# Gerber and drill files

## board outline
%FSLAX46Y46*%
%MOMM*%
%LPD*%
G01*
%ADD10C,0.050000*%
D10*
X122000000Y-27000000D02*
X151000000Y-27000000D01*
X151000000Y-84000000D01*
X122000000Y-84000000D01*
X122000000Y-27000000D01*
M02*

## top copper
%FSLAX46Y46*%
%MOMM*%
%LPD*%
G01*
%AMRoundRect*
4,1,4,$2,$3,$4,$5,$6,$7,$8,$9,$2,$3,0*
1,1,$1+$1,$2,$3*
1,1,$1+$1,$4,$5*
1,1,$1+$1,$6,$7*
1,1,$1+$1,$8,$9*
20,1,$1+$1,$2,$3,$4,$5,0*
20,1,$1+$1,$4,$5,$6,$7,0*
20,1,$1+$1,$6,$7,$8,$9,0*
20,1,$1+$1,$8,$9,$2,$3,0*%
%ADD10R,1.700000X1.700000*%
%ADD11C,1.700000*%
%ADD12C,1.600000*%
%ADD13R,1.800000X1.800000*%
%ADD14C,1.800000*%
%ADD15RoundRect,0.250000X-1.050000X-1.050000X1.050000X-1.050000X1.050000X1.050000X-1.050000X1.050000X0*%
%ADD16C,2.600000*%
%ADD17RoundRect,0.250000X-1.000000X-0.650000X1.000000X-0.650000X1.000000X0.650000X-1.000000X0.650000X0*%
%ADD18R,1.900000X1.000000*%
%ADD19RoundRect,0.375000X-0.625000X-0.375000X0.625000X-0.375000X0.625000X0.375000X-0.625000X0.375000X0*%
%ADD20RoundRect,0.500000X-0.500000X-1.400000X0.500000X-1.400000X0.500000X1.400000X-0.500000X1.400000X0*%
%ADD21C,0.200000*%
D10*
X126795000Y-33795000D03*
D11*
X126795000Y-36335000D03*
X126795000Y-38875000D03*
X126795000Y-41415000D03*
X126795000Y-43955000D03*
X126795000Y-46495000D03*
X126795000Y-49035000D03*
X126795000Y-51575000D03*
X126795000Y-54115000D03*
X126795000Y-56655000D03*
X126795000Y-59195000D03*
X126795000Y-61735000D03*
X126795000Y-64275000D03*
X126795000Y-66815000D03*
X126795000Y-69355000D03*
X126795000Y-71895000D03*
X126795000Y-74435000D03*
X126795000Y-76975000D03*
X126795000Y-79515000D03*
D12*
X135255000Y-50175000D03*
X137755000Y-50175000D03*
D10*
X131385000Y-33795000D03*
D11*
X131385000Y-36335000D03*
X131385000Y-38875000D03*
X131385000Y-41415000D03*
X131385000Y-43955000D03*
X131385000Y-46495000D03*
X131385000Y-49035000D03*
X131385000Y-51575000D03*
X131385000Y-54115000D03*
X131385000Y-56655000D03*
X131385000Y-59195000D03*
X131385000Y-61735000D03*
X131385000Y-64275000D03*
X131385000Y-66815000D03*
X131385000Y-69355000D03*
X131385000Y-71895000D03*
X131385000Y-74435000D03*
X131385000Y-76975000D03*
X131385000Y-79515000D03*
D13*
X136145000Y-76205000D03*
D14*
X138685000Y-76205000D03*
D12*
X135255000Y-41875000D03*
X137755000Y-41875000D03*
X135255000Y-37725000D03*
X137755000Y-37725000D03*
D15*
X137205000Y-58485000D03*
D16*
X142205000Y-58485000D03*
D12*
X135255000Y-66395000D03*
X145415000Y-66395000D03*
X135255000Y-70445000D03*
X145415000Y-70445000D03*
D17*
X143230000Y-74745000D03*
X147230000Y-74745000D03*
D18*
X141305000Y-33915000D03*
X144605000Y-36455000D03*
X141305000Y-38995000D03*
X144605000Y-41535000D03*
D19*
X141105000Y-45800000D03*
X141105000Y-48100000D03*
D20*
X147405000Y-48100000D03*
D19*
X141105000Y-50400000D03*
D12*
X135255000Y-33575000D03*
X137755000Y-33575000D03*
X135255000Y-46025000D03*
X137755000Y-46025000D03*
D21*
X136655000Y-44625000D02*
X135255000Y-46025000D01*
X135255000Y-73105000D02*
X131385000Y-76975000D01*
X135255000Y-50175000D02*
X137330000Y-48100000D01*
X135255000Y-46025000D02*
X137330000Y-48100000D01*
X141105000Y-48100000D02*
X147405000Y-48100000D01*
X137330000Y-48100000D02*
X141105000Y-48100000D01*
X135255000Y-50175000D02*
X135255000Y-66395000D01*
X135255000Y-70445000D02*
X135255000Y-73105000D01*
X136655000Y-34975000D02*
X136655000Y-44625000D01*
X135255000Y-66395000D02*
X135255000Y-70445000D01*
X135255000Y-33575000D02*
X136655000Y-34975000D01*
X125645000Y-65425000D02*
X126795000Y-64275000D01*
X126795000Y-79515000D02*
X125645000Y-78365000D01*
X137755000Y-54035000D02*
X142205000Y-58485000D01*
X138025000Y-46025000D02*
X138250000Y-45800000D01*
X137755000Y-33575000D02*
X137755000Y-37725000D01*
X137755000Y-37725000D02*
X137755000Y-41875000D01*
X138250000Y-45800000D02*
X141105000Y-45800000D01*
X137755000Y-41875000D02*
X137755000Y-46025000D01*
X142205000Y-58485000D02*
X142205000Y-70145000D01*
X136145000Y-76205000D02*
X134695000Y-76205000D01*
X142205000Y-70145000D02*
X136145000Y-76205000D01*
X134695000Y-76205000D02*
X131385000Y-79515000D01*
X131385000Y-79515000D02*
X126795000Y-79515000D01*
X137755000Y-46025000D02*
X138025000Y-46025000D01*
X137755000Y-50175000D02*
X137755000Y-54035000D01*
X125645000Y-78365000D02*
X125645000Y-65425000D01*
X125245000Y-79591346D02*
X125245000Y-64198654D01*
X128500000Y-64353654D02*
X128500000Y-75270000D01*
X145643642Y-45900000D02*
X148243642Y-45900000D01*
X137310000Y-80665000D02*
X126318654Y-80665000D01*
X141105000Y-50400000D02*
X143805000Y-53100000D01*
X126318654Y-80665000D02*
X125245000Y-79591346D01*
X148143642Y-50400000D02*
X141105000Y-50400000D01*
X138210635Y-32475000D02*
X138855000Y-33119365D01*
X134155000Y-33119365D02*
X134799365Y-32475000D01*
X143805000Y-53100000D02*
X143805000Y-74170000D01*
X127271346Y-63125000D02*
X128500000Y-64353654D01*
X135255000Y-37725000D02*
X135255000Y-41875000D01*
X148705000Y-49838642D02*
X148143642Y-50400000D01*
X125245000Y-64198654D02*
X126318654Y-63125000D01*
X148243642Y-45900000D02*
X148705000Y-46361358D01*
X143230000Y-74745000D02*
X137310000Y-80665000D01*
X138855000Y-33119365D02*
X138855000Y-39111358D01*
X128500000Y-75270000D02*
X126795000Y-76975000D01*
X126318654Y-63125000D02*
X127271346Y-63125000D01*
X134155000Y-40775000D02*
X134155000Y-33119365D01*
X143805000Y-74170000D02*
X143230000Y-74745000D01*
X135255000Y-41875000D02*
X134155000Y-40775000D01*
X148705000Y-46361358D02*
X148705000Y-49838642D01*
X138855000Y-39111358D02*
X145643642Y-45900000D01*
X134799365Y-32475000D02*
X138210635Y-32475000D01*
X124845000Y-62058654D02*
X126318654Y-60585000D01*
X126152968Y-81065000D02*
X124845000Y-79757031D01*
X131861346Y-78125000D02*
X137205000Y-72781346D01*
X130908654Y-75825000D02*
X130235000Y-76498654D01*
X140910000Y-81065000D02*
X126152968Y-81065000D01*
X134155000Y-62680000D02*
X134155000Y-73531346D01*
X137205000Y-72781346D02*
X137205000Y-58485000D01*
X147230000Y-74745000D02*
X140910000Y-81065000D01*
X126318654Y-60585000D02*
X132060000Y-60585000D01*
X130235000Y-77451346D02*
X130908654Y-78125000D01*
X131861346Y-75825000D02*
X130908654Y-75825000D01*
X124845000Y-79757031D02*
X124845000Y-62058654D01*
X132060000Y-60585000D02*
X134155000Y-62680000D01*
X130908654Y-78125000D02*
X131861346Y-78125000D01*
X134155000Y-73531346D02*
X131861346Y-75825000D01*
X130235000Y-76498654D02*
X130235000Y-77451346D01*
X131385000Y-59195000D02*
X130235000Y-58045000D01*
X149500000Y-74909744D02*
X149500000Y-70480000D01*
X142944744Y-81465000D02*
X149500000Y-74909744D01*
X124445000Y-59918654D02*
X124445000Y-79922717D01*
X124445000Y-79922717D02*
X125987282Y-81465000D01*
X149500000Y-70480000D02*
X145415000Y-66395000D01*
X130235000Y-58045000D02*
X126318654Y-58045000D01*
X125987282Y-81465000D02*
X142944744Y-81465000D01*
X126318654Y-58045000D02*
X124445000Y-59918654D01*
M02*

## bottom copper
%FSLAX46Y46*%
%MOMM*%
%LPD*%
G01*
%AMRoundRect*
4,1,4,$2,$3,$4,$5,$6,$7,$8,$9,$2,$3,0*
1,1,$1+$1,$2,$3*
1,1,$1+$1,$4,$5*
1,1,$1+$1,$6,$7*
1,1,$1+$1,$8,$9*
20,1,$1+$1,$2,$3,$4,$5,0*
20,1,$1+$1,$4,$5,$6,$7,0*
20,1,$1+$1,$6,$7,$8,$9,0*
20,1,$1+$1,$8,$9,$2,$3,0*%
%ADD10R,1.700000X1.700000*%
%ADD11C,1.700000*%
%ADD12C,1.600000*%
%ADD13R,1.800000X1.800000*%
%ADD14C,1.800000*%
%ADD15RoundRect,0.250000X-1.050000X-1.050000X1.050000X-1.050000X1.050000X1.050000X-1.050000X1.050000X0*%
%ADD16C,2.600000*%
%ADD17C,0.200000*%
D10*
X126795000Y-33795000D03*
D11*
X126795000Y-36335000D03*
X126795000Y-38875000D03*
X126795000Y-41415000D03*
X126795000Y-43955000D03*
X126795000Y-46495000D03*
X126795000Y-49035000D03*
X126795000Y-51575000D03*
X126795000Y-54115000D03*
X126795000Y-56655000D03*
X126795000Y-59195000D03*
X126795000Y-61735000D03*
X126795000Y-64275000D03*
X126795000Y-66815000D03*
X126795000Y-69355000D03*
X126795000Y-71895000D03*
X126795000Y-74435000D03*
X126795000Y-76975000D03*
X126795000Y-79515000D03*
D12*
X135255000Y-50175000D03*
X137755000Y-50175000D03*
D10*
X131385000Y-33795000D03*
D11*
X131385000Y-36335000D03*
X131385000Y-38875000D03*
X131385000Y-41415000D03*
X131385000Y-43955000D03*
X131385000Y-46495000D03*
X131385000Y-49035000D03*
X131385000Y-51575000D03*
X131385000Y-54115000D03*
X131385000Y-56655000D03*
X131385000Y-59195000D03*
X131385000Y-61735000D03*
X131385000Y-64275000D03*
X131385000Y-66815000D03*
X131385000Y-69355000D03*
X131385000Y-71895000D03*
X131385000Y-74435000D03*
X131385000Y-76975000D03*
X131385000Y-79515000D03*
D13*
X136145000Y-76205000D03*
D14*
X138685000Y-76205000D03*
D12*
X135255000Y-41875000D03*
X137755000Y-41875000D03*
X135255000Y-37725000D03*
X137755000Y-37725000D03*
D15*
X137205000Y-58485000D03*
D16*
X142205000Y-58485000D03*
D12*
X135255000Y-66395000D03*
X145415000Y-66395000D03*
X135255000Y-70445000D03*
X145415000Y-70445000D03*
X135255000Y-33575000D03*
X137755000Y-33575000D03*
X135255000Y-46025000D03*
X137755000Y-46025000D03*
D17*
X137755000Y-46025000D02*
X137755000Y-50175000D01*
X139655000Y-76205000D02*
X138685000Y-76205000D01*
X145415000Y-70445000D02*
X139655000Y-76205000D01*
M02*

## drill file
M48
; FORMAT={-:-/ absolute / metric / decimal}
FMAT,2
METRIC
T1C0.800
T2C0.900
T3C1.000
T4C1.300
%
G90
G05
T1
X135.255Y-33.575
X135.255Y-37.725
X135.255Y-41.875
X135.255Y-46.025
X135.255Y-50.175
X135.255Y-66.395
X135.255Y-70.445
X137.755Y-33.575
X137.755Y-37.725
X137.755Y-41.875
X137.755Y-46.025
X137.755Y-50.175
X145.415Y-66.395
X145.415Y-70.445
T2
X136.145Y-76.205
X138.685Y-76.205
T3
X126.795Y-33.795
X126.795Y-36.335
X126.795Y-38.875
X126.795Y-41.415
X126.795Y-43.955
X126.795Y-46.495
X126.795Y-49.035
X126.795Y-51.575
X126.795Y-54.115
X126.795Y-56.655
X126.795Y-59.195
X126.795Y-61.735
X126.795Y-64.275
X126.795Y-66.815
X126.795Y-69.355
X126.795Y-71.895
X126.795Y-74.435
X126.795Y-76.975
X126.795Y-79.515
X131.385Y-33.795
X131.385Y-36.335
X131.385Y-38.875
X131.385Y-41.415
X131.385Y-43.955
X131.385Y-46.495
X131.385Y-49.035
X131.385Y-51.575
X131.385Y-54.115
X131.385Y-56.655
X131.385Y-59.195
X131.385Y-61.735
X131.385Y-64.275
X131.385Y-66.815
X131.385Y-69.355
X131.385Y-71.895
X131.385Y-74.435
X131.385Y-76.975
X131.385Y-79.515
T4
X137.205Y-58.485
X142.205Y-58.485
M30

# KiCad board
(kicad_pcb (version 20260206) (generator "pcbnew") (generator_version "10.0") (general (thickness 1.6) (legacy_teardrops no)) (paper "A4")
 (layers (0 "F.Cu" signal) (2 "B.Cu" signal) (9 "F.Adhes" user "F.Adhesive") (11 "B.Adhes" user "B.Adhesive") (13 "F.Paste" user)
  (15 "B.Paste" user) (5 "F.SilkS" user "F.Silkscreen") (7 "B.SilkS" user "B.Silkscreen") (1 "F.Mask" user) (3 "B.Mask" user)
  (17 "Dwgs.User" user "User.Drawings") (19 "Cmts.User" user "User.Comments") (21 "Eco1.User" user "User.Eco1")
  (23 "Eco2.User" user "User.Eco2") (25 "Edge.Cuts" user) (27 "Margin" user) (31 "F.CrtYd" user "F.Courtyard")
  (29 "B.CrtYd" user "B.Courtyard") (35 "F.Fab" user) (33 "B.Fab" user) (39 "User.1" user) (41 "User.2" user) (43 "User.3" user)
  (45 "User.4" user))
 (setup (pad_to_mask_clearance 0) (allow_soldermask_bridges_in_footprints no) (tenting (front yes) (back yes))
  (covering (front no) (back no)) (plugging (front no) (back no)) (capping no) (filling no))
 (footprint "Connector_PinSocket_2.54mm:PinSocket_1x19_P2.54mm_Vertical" (layer "F.Cu") (at 126.795 33.795)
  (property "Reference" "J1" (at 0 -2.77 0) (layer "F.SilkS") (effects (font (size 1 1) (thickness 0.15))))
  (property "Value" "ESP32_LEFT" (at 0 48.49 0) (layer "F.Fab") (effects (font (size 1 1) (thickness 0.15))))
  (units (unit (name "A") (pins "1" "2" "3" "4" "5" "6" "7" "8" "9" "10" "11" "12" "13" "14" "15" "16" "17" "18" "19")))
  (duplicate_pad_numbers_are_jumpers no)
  (pad "1" thru_hole rect (at 0 0) (size 1.7 1.7) (drill 1) (layers "*.Cu" "*.Mask") (remove_unused_layers no)
   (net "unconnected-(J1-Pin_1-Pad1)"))
  (pad "2" thru_hole circle (at 0 2.54) (size 1.7 1.7) (drill 1) (layers "*.Cu" "*.Mask") (remove_unused_layers no)
   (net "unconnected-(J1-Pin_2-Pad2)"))
  (pad "3" thru_hole circle (at 0 5.08) (size 1.7 1.7) (drill 1) (layers "*.Cu" "*.Mask") (remove_unused_layers no)
   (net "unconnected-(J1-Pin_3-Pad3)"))
  (pad "4" thru_hole circle (at 0 7.62) (size 1.7 1.7) (drill 1) (layers "*.Cu" "*.Mask") (remove_unused_layers no)
   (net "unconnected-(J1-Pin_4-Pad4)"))
  (pad "5" thru_hole circle (at 0 10.16) (size 1.7 1.7) (drill 1) (layers "*.Cu" "*.Mask") (remove_unused_layers no)
   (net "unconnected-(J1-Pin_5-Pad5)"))
  (pad "6" thru_hole circle (at 0 12.7) (size 1.7 1.7) (drill 1) (layers "*.Cu" "*.Mask") (remove_unused_layers no)
   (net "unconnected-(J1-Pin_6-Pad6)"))
  (pad "7" thru_hole circle (at 0 15.24) (size 1.7 1.7) (drill 1) (layers "*.Cu" "*.Mask") (remove_unused_layers no)
   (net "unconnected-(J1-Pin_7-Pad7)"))
  (pad "8" thru_hole circle (at 0 17.78) (size 1.7 1.7) (drill 1) (layers "*.Cu" "*.Mask") (remove_unused_layers no)
   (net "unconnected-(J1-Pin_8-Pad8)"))
  (pad "9" thru_hole circle (at 0 20.32) (size 1.7 1.7) (drill 1) (layers "*.Cu" "*.Mask") (remove_unused_layers no)
   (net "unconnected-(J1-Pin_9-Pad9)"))
  (pad "10" thru_hole circle (at 0 22.86) (size 1.7 1.7) (drill 1) (layers "*.Cu" "*.Mask") (remove_unused_layers no)
   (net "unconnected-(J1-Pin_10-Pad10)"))
  (pad "11" thru_hole circle (at 0 25.4) (size 1.7 1.7) (drill 1) (layers "*.Cu" "*.Mask") (remove_unused_layers no)
   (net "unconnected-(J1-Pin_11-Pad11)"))
  (pad "12" thru_hole circle (at 0 27.94) (size 1.7 1.7) (drill 1) (layers "*.Cu" "*.Mask") (remove_unused_layers no)
   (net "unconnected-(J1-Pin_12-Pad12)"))
  (pad "13" thru_hole circle (at 0 30.48) (size 1.7 1.7) (drill 1) (layers "*.Cu" "*.Mask") (remove_unused_layers no) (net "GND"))
  (pad "14" thru_hole circle (at 0 33.02) (size 1.7 1.7) (drill 1) (layers "*.Cu" "*.Mask") (remove_unused_layers no)
   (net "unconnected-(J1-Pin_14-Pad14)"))
  (pad "15" thru_hole circle (at 0 35.56) (size 1.7 1.7) (drill 1) (layers "*.Cu" "*.Mask") (remove_unused_layers no)
   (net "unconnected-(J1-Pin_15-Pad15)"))
  (pad "16" thru_hole circle (at 0 38.1) (size 1.7 1.7) (drill 1) (layers "*.Cu" "*.Mask") (remove_unused_layers no)
   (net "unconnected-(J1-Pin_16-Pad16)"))
  (pad "17" thru_hole circle (at 0 40.64) (size 1.7 1.7) (drill 1) (layers "*.Cu" "*.Mask") (remove_unused_layers no)
   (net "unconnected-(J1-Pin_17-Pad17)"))
  (pad "18" thru_hole circle (at 0 43.18) (size 1.7 1.7) (drill 1) (layers "*.Cu" "*.Mask") (remove_unused_layers no) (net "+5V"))
  (pad "19" thru_hole circle (at 0 45.72) (size 1.7 1.7) (drill 1) (layers "*.Cu" "*.Mask") (remove_unused_layers no) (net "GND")))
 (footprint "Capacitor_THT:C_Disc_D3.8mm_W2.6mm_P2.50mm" (layer "F.Cu") (at 135.255 50.175)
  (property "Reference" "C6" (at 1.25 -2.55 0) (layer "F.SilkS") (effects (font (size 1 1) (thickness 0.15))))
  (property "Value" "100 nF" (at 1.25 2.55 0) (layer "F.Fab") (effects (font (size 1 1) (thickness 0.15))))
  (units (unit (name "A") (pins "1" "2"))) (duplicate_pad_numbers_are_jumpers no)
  (pad "1" thru_hole circle (at 0 0) (size 1.6 1.6) (drill 0.8) (layers "*.Cu" "*.Mask") (remove_unused_layers no) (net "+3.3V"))
  (pad "2" thru_hole circle (at 2.5 0) (size 1.6 1.6) (drill 0.8) (layers "*.Cu" "*.Mask") (remove_unused_layers no) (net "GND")))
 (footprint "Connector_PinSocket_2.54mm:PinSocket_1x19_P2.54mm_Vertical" (layer "F.Cu") (at 131.385 33.795)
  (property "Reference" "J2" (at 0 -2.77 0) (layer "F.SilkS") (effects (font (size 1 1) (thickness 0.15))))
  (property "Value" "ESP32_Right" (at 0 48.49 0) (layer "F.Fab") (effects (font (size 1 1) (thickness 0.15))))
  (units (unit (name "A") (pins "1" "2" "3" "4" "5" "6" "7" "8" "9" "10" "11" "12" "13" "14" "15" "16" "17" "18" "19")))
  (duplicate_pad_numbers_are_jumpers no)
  (pad "1" thru_hole rect (at 0 0) (size 1.7 1.7) (drill 1) (layers "*.Cu" "*.Mask") (remove_unused_layers no)
   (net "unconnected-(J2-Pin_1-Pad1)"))
  (pad "2" thru_hole circle (at 0 2.54) (size 1.7 1.7) (drill 1) (layers "*.Cu" "*.Mask") (remove_unused_layers no)
   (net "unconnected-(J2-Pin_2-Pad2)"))
  (pad "3" thru_hole circle (at 0 5.08) (size 1.7 1.7) (drill 1) (layers "*.Cu" "*.Mask") (remove_unused_layers no)
   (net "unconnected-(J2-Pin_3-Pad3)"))
  (pad "4" thru_hole circle (at 0 7.62) (size 1.7 1.7) (drill 1) (layers "*.Cu" "*.Mask") (remove_unused_layers no)
   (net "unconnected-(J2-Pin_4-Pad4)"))
  (pad "5" thru_hole circle (at 0 10.16) (size 1.7 1.7) (drill 1) (layers "*.Cu" "*.Mask") (remove_unused_layers no)
   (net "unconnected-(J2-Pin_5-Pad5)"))
  (pad "6" thru_hole circle (at 0 12.7) (size 1.7 1.7) (drill 1) (layers "*.Cu" "*.Mask") (remove_unused_layers no)
   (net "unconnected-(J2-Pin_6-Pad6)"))
  (pad "7" thru_hole circle (at 0 15.24) (size 1.7 1.7) (drill 1) (layers "*.Cu" "*.Mask") (remove_unused_layers no)
   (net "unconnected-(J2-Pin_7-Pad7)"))
  (pad "8" thru_hole circle (at 0 17.78) (size 1.7 1.7) (drill 1) (layers "*.Cu" "*.Mask") (remove_unused_layers no)
   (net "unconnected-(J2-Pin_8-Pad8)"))
  (pad "9" thru_hole circle (at 0 20.32) (size 1.7 1.7) (drill 1) (layers "*.Cu" "*.Mask") (remove_unused_layers no)
   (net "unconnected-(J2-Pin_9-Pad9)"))
  (pad "10" thru_hole circle (at 0 22.86) (size 1.7 1.7) (drill 1) (layers "*.Cu" "*.Mask") (remove_unused_layers no)
   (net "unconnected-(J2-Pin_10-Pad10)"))
  (pad "11" thru_hole circle (at 0 25.4) (size 1.7 1.7) (drill 1) (layers "*.Cu" "*.Mask") (remove_unused_layers no) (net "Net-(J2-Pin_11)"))
  (pad "12" thru_hole circle (at 0 27.94) (size 1.7 1.7) (drill 1) (layers "*.Cu" "*.Mask") (remove_unused_layers no)
   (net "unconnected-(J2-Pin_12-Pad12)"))
  (pad "13" thru_hole circle (at 0 30.48) (size 1.7 1.7) (drill 1) (layers "*.Cu" "*.Mask") (remove_unused_layers no)
   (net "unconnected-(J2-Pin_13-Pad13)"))
  (pad "14" thru_hole circle (at 0 33.02) (size 1.7 1.7) (drill 1) (layers "*.Cu" "*.Mask") (remove_unused_layers no)
   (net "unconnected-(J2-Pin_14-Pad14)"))
  (pad "15" thru_hole circle (at 0 35.56) (size 1.7 1.7) (drill 1) (layers "*.Cu" "*.Mask") (remove_unused_layers no)
   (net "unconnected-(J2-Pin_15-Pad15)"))
  (pad "16" thru_hole circle (at 0 38.1) (size 1.7 1.7) (drill 1) (layers "*.Cu" "*.Mask") (remove_unused_layers no)
   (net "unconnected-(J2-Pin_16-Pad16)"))
  (pad "17" thru_hole circle (at 0 40.64) (size 1.7 1.7) (drill 1) (layers "*.Cu" "*.Mask") (remove_unused_layers no)
   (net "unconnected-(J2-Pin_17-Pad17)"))
  (pad "18" thru_hole circle (at 0 43.18) (size 1.7 1.7) (drill 1) (layers "*.Cu" "*.Mask") (remove_unused_layers no) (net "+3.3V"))
  (pad "19" thru_hole circle (at 0 45.72) (size 1.7 1.7) (drill 1) (layers "*.Cu" "*.Mask") (remove_unused_layers no) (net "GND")))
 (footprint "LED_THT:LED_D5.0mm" (layer "F.Cu") (at 136.145 76.205)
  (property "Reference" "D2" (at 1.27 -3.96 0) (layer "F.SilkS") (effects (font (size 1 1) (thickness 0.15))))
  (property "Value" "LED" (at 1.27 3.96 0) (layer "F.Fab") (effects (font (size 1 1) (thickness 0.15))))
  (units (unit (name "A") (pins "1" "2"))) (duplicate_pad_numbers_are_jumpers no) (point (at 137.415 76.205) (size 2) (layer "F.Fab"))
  (pad "1" thru_hole rect (at 0 0) (size 1.8 1.8) (drill 0.9) (layers "*.Cu" "*.Mask") (remove_unused_layers no) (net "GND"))
  (pad "2" thru_hole circle (at 2.54 0) (size 1.8 1.8) (drill 0.9) (layers "*.Cu" "*.Mask") (remove_unused_layers no) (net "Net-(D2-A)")))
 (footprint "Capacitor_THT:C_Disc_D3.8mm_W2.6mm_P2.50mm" (layer "F.Cu") (at 135.255 41.875)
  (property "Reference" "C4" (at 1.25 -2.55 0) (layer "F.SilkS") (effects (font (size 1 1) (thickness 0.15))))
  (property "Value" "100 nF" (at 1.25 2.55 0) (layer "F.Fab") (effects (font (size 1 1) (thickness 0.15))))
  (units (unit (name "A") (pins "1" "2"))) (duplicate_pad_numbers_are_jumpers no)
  (pad "1" thru_hole circle (at 0 0) (size 1.6 1.6) (drill 0.8) (layers "*.Cu" "*.Mask") (remove_unused_layers no) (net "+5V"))
  (pad "2" thru_hole circle (at 2.5 0) (size 1.6 1.6) (drill 0.8) (layers "*.Cu" "*.Mask") (remove_unused_layers no) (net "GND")))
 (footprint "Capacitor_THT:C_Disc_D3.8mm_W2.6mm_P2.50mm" (layer "F.Cu") (at 135.255 37.725)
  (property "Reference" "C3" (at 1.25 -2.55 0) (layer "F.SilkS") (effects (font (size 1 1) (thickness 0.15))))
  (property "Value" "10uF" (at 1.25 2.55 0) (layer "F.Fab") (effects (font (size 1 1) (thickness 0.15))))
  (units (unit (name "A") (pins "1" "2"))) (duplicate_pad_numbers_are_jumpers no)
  (pad "1" thru_hole circle (at 0 0) (size 1.6 1.6) (drill 0.8) (layers "*.Cu" "*.Mask") (remove_unused_layers no) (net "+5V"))
  (pad "2" thru_hole circle (at 2.5 0) (size 1.6 1.6) (drill 0.8) (layers "*.Cu" "*.Mask") (remove_unused_layers no) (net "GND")))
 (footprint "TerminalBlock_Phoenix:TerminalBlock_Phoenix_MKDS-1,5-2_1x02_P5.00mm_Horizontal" (layer "F.Cu") (at 137.205 58.485)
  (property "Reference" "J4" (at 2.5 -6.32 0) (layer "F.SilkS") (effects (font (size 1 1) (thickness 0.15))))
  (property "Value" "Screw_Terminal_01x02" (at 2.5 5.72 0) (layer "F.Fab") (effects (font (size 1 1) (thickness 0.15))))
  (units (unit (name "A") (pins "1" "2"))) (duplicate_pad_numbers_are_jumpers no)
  (pad "1" thru_hole roundrect (at 0 0) (size 2.6 2.6) (drill 1.3) (layers "*.Cu" "*.Mask") (remove_unused_layers no)
   (roundrect_rratio 0.096154) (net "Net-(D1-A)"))
  (pad "2" thru_hole circle (at 5 0) (size 2.6 2.6) (drill 1.3) (layers "*.Cu" "*.Mask") (remove_unused_layers no) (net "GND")))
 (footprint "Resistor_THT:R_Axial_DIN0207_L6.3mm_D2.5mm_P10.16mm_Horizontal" (layer "F.Cu") (at 135.255 66.395)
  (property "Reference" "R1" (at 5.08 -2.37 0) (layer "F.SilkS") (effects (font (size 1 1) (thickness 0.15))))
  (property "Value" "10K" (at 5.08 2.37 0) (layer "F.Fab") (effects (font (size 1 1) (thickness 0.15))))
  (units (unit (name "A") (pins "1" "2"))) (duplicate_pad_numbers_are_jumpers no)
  (pad "1" thru_hole circle (at 0 0) (size 1.6 1.6) (drill 0.8) (layers "*.Cu" "*.Mask") (remove_unused_layers no) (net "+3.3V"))
  (pad "2" thru_hole circle (at 10.16 0) (size 1.6 1.6) (drill 0.8) (layers "*.Cu" "*.Mask") (remove_unused_layers no)
   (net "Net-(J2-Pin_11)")))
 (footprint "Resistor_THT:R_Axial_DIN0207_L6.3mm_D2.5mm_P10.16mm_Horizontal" (layer "F.Cu") (at 135.255 70.445)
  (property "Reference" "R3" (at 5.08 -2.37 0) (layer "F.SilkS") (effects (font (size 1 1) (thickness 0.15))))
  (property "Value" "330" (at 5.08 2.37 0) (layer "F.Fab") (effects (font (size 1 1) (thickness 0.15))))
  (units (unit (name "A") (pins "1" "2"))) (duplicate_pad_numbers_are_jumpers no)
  (pad "1" thru_hole circle (at 0 0) (size 1.6 1.6) (drill 0.8) (layers "*.Cu" "*.Mask") (remove_unused_layers no) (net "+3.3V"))
  (pad "2" thru_hole circle (at 10.16 0) (size 1.6 1.6) (drill 0.8) (layers "*.Cu" "*.Mask") (remove_unused_layers no) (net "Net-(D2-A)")))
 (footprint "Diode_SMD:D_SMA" (layer "F.Cu") (at 145.23 74.745)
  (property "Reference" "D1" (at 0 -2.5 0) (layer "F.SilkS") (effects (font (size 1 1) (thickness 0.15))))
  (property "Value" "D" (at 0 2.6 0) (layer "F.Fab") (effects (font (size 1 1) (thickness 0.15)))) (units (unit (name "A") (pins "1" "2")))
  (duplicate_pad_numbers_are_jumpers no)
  (pad "1" smd roundrect (at -2 0) (size 2.5 1.8) (layers "F.Cu" "F.Mask" "F.Paste") (roundrect_rratio 0.1388888889) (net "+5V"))
  (pad "2" smd roundrect (at 2 0) (size 2.5 1.8) (layers "F.Cu" "F.Mask" "F.Paste") (roundrect_rratio 0.1388888889) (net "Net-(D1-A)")))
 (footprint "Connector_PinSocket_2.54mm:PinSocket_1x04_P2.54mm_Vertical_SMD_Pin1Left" (layer "F.Cu") (at 142.955 37.725)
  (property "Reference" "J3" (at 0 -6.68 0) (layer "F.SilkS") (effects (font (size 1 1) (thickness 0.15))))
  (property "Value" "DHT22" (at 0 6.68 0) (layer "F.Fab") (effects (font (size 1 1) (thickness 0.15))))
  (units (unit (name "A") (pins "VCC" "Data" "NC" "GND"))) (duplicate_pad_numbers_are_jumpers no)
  (pad "1" smd rect (at -1.65 -3.81) (size 1.9 1) (layers "F.Cu" "F.Mask" "F.Paste"))
  (pad "2" smd rect (at 1.65 -1.27) (size 1.9 1) (layers "F.Cu" "F.Mask" "F.Paste"))
  (pad "3" smd rect (at -1.65 1.27) (size 1.9 1) (layers "F.Cu" "F.Mask" "F.Paste"))
  (pad "4" smd rect (at 1.65 3.81) (size 1.9 1) (layers "F.Cu" "F.Mask" "F.Paste")))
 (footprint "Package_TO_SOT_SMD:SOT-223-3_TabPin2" (layer "F.Cu") (at 144.255 48.1)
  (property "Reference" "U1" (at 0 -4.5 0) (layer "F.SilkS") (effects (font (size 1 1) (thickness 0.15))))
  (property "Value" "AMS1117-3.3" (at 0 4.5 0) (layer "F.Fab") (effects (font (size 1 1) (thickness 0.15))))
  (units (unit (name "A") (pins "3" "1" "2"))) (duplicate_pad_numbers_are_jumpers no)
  (pad "1" smd roundrect (at -3.15 -2.3) (size 2 1.5) (layers "F.Cu" "F.Mask" "F.Paste") (roundrect_rratio 0.25) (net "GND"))
  (pad "2" smd roundrect (at -3.15 0) (size 2 1.5) (layers "F.Cu" "F.Mask" "F.Paste") (roundrect_rratio 0.25) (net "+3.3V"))
  (pad "2" smd roundrect (at 3.15 0) (size 2 3.8) (layers "F.Cu" "F.Mask" "F.Paste") (roundrect_rratio 0.25) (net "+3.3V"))
  (pad "3" smd roundrect (at -3.15 2.3) (size 2 1.5) (layers "F.Cu" "F.Mask" "F.Paste") (roundrect_rratio 0.25) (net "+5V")))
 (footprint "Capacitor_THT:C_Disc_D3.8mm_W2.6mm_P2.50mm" (layer "F.Cu") (at 135.255 33.575)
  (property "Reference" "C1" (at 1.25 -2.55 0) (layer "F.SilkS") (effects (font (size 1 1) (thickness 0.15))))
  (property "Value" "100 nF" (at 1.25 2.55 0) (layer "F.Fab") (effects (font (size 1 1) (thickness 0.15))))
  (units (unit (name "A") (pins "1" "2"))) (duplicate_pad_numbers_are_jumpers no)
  (pad "1" thru_hole circle (at 0 0) (size 1.6 1.6) (drill 0.8) (layers "*.Cu" "*.Mask") (remove_unused_layers no) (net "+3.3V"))
  (pad "2" thru_hole circle (at 2.5 0) (size 1.6 1.6) (drill 0.8) (layers "*.Cu" "*.Mask") (remove_unused_layers no) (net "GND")))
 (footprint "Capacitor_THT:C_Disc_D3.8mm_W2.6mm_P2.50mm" (layer "F.Cu") (at 135.255 46.025)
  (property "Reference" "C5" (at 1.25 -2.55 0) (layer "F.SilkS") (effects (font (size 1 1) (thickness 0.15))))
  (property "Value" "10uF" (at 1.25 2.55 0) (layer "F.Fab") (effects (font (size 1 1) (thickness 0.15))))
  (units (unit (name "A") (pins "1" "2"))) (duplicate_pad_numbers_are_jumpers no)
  (pad "1" thru_hole circle (at 0 0) (size 1.6 1.6) (drill 0.8) (layers "*.Cu" "*.Mask") (remove_unused_layers no) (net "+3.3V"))
  (pad "2" thru_hole circle (at 2.5 0) (size 1.6 1.6) (drill 0.8) (layers "*.Cu" "*.Mask") (remove_unused_layers no) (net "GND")))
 (gr_rect (start 122 27) (end 151 84) (stroke (width 0.05) (type default)) (fill no) (layer "Edge.Cuts"))
 (segment (start 136.655 44.625) (end 135.255 46.025) (width 0.2) (layer "F.Cu") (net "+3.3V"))
 (segment (start 135.255 73.105) (end 131.385 76.975) (width 0.2) (layer "F.Cu") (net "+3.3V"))
 (segment (start 135.255 50.175) (end 137.33 48.1) (width 0.2) (layer "F.Cu") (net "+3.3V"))
 (segment (start 135.255 46.025) (end 137.33 48.1) (width 0.2) (layer "F.Cu") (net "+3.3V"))
 (segment (start 141.105 48.1) (end 147.405 48.1) (width 0.2) (layer "F.Cu") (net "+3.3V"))
 (segment (start 137.33 48.1) (end 141.105 48.1) (width 0.2) (layer "F.Cu") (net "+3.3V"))
 (segment (start 135.255 50.175) (end 135.255 66.395) (width 0.2) (layer "F.Cu") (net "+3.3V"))
 (segment (start 135.255 70.445) (end 135.255 73.105) (width 0.2) (layer "F.Cu") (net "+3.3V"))
 (segment (start 136.655 34.975) (end 136.655 44.625) (width 0.2) (layer "F.Cu") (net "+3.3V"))
 (segment (start 135.255 66.395) (end 135.255 70.445) (width 0.2) (layer "F.Cu") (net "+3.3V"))
 (segment (start 135.255 33.575) (end 136.655 34.975) (width 0.2) (layer "F.Cu") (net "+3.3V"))
 (segment (start 125.645 65.425) (end 126.795 64.275) (width 0.2) (layer "F.Cu") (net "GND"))
 (segment (start 126.795 79.515) (end 125.645 78.365) (width 0.2) (layer "F.Cu") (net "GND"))
 (segment (start 137.755 54.035) (end 142.205 58.485) (width 0.2) (layer "F.Cu") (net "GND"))
 (segment (start 138.025 46.025) (end 138.25 45.8) (width 0.2) (layer "F.Cu") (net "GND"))
 (segment (start 137.755 33.575) (end 137.755 37.725) (width 0.2) (layer "F.Cu") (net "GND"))
 (segment (start 137.755 37.725) (end 137.755 41.875) (width 0.2) (layer "F.Cu") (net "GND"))
 (segment (start 138.25 45.8) (end 141.105 45.8) (width 0.2) (layer "F.Cu") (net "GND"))
 (segment (start 137.755 41.875) (end 137.755 46.025) (width 0.2) (layer "F.Cu") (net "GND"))
 (segment (start 142.205 58.485) (end 142.205 70.145) (width 0.2) (layer "F.Cu") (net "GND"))
 (segment (start 136.145 76.205) (end 134.695 76.205) (width 0.2) (layer "F.Cu") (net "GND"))
 (segment (start 142.205 70.145) (end 136.145 76.205) (width 0.2) (layer "F.Cu") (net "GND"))
 (segment (start 134.695 76.205) (end 131.385 79.515) (width 0.2) (layer "F.Cu") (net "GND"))
 (segment (start 131.385 79.515) (end 126.795 79.515) (width 0.2) (layer "F.Cu") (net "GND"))
 (segment (start 137.755 46.025) (end 138.025 46.025) (width 0.2) (layer "F.Cu") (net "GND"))
 (segment (start 137.755 50.175) (end 137.755 54.035) (width 0.2) (layer "F.Cu") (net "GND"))
 (segment (start 125.645 78.365) (end 125.645 65.425) (width 0.2) (layer "F.Cu") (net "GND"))
 (segment (start 137.755 46.025) (end 137.755 50.175) (width 0.2) (layer "B.Cu") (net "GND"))
 (segment (start 125.245 79.591346) (end 125.245 64.198654) (width 0.2) (layer "F.Cu") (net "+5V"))
 (segment (start 128.5 64.353654) (end 128.5 75.27) (width 0.2) (layer "F.Cu") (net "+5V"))
 (segment (start 145.643642 45.9) (end 148.243642 45.9) (width 0.2) (layer "F.Cu") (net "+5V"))
 (segment (start 137.31 80.665) (end 126.318654 80.665) (width 0.2) (layer "F.Cu") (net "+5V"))
 (segment (start 141.105 50.4) (end 143.805 53.1) (width 0.2) (layer "F.Cu") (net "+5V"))
 (segment (start 126.318654 80.665) (end 125.245 79.591346) (width 0.2) (layer "F.Cu") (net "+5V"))
 (segment (start 148.143642 50.4) (end 141.105 50.4) (width 0.2) (layer "F.Cu") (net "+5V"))
 (segment (start 138.210635 32.475) (end 138.855 33.119365) (width 0.2) (layer "F.Cu") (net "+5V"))
 (segment (start 134.155 33.119365) (end 134.799365 32.475) (width 0.2) (layer "F.Cu") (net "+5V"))
 (segment (start 143.805 53.1) (end 143.805 74.17) (width 0.2) (layer "F.Cu") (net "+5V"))
 (segment (start 127.271346 63.125) (end 128.5 64.353654) (width 0.2) (layer "F.Cu") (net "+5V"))
 (segment (start 135.255 37.725) (end 135.255 41.875) (width 0.2) (layer "F.Cu") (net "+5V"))
 (segment (start 148.705 49.838642) (end 148.143642 50.4) (width 0.2) (layer "F.Cu") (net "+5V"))
 (segment (start 125.245 64.198654) (end 126.318654 63.125) (width 0.2) (layer "F.Cu") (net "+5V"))
 (segment (start 148.243642 45.9) (end 148.705 46.361358) (width 0.2) (layer "F.Cu") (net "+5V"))
 (segment (start 143.23 74.745) (end 137.31 80.665) (width 0.2) (layer "F.Cu") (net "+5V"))
 (segment (start 138.855 33.119365) (end 138.855 39.111358) (width 0.2) (layer "F.Cu") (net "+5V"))
 (segment (start 128.5 75.27) (end 126.795 76.975) (width 0.2) (layer "F.Cu") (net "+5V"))
 (segment (start 126.318654 63.125) (end 127.271346 63.125) (width 0.2) (layer "F.Cu") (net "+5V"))
 (segment (start 134.155 40.775) (end 134.155 33.119365) (width 0.2) (layer "F.Cu") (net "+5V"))
 (segment (start 143.805 74.17) (end 143.23 74.745) (width 0.2) (layer "F.Cu") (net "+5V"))
 (segment (start 135.255 41.875) (end 134.155 40.775) (width 0.2) (layer "F.Cu") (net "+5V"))
 (segment (start 148.705 46.361358) (end 148.705 49.838642) (width 0.2) (layer "F.Cu") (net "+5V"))
 (segment (start 138.855 39.111358) (end 145.643642 45.9) (width 0.2) (layer "F.Cu") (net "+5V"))
 (segment (start 134.799365 32.475) (end 138.210635 32.475) (width 0.2) (layer "F.Cu") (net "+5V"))
 (segment (start 124.845 62.058654) (end 126.318654 60.585) (width 0.2) (layer "F.Cu") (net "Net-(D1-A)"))
 (segment (start 126.152968 81.065) (end 124.845 79.757031) (width 0.2) (layer "F.Cu") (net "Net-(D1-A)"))
 (segment (start 131.861346 78.125) (end 137.205 72.781346) (width 0.2) (layer "F.Cu") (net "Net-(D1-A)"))
 (segment (start 130.908654 75.825) (end 130.235 76.498654) (width 0.2) (layer "F.Cu") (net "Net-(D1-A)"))
 (segment (start 140.91 81.065) (end 126.152968 81.065) (width 0.2) (layer "F.Cu") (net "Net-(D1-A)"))
 (segment (start 134.155 62.68) (end 134.155 73.531346) (width 0.2) (layer "F.Cu") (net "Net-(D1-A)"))
 (segment (start 137.205 72.781346) (end 137.205 58.485) (width 0.2) (layer "F.Cu") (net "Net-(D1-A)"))
 (segment (start 147.23 74.745) (end 140.91 81.065) (width 0.2) (layer "F.Cu") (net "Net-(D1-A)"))
 (segment (start 126.318654 60.585) (end 132.06 60.585) (width 0.2) (layer "F.Cu") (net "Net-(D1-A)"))
 (segment (start 130.235 77.451346) (end 130.908654 78.125) (width 0.2) (layer "F.Cu") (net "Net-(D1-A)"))
 (segment (start 131.861346 75.825) (end 130.908654 75.825) (width 0.2) (layer "F.Cu") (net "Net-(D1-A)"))
 (segment (start 124.845 79.757031) (end 124.845 62.058654) (width 0.2) (layer "F.Cu") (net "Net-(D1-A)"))
 (segment (start 132.06 60.585) (end 134.155 62.68) (width 0.2) (layer "F.Cu") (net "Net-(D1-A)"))
 (segment (start 130.908654 78.125) (end 131.861346 78.125) (width 0.2) (layer "F.Cu") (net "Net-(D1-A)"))
 (segment (start 134.155 73.531346) (end 131.861346 75.825) (width 0.2) (layer "F.Cu") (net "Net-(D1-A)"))
 (segment (start 130.235 76.498654) (end 130.235 77.451346) (width 0.2) (layer "F.Cu") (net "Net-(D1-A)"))
 (segment (start 139.655 76.205) (end 138.685 76.205) (width 0.2) (layer "B.Cu") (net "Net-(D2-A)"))
 (segment (start 145.415 70.445) (end 139.655 76.205) (width 0.2) (layer "B.Cu") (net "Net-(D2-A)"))
 (segment (start 131.385 59.195) (end 130.235 58.045) (width 0.2) (layer "F.Cu") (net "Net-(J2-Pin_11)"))
 (segment (start 149.5 74.909744) (end 149.5 70.48) (width 0.2) (layer "F.Cu") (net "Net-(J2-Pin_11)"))
 (segment (start 142.944744 81.465) (end 149.5 74.909744) (width 0.2) (layer "F.Cu") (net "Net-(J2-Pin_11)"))
 (segment (start 124.445 59.918654) (end 124.445 79.922717) (width 0.2) (layer "F.Cu") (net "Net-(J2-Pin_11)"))
 (segment (start 124.445 79.922717) (end 125.987282 81.465) (width 0.2) (layer "F.Cu") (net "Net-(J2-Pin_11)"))
 (segment (start 149.5 70.48) (end 145.415 66.395) (width 0.2) (layer "F.Cu") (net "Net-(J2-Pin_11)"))
 (segment (start 130.235 58.045) (end 126.318654 58.045) (width 0.2) (layer "F.Cu") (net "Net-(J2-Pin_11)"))
 (segment (start 125.987282 81.465) (end 142.944744 81.465) (width 0.2) (layer "F.Cu") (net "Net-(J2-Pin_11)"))
 (segment (start 126.318654 58.045) (end 124.445 59.918654) (width 0.2) (layer "F.Cu") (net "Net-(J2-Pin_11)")))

